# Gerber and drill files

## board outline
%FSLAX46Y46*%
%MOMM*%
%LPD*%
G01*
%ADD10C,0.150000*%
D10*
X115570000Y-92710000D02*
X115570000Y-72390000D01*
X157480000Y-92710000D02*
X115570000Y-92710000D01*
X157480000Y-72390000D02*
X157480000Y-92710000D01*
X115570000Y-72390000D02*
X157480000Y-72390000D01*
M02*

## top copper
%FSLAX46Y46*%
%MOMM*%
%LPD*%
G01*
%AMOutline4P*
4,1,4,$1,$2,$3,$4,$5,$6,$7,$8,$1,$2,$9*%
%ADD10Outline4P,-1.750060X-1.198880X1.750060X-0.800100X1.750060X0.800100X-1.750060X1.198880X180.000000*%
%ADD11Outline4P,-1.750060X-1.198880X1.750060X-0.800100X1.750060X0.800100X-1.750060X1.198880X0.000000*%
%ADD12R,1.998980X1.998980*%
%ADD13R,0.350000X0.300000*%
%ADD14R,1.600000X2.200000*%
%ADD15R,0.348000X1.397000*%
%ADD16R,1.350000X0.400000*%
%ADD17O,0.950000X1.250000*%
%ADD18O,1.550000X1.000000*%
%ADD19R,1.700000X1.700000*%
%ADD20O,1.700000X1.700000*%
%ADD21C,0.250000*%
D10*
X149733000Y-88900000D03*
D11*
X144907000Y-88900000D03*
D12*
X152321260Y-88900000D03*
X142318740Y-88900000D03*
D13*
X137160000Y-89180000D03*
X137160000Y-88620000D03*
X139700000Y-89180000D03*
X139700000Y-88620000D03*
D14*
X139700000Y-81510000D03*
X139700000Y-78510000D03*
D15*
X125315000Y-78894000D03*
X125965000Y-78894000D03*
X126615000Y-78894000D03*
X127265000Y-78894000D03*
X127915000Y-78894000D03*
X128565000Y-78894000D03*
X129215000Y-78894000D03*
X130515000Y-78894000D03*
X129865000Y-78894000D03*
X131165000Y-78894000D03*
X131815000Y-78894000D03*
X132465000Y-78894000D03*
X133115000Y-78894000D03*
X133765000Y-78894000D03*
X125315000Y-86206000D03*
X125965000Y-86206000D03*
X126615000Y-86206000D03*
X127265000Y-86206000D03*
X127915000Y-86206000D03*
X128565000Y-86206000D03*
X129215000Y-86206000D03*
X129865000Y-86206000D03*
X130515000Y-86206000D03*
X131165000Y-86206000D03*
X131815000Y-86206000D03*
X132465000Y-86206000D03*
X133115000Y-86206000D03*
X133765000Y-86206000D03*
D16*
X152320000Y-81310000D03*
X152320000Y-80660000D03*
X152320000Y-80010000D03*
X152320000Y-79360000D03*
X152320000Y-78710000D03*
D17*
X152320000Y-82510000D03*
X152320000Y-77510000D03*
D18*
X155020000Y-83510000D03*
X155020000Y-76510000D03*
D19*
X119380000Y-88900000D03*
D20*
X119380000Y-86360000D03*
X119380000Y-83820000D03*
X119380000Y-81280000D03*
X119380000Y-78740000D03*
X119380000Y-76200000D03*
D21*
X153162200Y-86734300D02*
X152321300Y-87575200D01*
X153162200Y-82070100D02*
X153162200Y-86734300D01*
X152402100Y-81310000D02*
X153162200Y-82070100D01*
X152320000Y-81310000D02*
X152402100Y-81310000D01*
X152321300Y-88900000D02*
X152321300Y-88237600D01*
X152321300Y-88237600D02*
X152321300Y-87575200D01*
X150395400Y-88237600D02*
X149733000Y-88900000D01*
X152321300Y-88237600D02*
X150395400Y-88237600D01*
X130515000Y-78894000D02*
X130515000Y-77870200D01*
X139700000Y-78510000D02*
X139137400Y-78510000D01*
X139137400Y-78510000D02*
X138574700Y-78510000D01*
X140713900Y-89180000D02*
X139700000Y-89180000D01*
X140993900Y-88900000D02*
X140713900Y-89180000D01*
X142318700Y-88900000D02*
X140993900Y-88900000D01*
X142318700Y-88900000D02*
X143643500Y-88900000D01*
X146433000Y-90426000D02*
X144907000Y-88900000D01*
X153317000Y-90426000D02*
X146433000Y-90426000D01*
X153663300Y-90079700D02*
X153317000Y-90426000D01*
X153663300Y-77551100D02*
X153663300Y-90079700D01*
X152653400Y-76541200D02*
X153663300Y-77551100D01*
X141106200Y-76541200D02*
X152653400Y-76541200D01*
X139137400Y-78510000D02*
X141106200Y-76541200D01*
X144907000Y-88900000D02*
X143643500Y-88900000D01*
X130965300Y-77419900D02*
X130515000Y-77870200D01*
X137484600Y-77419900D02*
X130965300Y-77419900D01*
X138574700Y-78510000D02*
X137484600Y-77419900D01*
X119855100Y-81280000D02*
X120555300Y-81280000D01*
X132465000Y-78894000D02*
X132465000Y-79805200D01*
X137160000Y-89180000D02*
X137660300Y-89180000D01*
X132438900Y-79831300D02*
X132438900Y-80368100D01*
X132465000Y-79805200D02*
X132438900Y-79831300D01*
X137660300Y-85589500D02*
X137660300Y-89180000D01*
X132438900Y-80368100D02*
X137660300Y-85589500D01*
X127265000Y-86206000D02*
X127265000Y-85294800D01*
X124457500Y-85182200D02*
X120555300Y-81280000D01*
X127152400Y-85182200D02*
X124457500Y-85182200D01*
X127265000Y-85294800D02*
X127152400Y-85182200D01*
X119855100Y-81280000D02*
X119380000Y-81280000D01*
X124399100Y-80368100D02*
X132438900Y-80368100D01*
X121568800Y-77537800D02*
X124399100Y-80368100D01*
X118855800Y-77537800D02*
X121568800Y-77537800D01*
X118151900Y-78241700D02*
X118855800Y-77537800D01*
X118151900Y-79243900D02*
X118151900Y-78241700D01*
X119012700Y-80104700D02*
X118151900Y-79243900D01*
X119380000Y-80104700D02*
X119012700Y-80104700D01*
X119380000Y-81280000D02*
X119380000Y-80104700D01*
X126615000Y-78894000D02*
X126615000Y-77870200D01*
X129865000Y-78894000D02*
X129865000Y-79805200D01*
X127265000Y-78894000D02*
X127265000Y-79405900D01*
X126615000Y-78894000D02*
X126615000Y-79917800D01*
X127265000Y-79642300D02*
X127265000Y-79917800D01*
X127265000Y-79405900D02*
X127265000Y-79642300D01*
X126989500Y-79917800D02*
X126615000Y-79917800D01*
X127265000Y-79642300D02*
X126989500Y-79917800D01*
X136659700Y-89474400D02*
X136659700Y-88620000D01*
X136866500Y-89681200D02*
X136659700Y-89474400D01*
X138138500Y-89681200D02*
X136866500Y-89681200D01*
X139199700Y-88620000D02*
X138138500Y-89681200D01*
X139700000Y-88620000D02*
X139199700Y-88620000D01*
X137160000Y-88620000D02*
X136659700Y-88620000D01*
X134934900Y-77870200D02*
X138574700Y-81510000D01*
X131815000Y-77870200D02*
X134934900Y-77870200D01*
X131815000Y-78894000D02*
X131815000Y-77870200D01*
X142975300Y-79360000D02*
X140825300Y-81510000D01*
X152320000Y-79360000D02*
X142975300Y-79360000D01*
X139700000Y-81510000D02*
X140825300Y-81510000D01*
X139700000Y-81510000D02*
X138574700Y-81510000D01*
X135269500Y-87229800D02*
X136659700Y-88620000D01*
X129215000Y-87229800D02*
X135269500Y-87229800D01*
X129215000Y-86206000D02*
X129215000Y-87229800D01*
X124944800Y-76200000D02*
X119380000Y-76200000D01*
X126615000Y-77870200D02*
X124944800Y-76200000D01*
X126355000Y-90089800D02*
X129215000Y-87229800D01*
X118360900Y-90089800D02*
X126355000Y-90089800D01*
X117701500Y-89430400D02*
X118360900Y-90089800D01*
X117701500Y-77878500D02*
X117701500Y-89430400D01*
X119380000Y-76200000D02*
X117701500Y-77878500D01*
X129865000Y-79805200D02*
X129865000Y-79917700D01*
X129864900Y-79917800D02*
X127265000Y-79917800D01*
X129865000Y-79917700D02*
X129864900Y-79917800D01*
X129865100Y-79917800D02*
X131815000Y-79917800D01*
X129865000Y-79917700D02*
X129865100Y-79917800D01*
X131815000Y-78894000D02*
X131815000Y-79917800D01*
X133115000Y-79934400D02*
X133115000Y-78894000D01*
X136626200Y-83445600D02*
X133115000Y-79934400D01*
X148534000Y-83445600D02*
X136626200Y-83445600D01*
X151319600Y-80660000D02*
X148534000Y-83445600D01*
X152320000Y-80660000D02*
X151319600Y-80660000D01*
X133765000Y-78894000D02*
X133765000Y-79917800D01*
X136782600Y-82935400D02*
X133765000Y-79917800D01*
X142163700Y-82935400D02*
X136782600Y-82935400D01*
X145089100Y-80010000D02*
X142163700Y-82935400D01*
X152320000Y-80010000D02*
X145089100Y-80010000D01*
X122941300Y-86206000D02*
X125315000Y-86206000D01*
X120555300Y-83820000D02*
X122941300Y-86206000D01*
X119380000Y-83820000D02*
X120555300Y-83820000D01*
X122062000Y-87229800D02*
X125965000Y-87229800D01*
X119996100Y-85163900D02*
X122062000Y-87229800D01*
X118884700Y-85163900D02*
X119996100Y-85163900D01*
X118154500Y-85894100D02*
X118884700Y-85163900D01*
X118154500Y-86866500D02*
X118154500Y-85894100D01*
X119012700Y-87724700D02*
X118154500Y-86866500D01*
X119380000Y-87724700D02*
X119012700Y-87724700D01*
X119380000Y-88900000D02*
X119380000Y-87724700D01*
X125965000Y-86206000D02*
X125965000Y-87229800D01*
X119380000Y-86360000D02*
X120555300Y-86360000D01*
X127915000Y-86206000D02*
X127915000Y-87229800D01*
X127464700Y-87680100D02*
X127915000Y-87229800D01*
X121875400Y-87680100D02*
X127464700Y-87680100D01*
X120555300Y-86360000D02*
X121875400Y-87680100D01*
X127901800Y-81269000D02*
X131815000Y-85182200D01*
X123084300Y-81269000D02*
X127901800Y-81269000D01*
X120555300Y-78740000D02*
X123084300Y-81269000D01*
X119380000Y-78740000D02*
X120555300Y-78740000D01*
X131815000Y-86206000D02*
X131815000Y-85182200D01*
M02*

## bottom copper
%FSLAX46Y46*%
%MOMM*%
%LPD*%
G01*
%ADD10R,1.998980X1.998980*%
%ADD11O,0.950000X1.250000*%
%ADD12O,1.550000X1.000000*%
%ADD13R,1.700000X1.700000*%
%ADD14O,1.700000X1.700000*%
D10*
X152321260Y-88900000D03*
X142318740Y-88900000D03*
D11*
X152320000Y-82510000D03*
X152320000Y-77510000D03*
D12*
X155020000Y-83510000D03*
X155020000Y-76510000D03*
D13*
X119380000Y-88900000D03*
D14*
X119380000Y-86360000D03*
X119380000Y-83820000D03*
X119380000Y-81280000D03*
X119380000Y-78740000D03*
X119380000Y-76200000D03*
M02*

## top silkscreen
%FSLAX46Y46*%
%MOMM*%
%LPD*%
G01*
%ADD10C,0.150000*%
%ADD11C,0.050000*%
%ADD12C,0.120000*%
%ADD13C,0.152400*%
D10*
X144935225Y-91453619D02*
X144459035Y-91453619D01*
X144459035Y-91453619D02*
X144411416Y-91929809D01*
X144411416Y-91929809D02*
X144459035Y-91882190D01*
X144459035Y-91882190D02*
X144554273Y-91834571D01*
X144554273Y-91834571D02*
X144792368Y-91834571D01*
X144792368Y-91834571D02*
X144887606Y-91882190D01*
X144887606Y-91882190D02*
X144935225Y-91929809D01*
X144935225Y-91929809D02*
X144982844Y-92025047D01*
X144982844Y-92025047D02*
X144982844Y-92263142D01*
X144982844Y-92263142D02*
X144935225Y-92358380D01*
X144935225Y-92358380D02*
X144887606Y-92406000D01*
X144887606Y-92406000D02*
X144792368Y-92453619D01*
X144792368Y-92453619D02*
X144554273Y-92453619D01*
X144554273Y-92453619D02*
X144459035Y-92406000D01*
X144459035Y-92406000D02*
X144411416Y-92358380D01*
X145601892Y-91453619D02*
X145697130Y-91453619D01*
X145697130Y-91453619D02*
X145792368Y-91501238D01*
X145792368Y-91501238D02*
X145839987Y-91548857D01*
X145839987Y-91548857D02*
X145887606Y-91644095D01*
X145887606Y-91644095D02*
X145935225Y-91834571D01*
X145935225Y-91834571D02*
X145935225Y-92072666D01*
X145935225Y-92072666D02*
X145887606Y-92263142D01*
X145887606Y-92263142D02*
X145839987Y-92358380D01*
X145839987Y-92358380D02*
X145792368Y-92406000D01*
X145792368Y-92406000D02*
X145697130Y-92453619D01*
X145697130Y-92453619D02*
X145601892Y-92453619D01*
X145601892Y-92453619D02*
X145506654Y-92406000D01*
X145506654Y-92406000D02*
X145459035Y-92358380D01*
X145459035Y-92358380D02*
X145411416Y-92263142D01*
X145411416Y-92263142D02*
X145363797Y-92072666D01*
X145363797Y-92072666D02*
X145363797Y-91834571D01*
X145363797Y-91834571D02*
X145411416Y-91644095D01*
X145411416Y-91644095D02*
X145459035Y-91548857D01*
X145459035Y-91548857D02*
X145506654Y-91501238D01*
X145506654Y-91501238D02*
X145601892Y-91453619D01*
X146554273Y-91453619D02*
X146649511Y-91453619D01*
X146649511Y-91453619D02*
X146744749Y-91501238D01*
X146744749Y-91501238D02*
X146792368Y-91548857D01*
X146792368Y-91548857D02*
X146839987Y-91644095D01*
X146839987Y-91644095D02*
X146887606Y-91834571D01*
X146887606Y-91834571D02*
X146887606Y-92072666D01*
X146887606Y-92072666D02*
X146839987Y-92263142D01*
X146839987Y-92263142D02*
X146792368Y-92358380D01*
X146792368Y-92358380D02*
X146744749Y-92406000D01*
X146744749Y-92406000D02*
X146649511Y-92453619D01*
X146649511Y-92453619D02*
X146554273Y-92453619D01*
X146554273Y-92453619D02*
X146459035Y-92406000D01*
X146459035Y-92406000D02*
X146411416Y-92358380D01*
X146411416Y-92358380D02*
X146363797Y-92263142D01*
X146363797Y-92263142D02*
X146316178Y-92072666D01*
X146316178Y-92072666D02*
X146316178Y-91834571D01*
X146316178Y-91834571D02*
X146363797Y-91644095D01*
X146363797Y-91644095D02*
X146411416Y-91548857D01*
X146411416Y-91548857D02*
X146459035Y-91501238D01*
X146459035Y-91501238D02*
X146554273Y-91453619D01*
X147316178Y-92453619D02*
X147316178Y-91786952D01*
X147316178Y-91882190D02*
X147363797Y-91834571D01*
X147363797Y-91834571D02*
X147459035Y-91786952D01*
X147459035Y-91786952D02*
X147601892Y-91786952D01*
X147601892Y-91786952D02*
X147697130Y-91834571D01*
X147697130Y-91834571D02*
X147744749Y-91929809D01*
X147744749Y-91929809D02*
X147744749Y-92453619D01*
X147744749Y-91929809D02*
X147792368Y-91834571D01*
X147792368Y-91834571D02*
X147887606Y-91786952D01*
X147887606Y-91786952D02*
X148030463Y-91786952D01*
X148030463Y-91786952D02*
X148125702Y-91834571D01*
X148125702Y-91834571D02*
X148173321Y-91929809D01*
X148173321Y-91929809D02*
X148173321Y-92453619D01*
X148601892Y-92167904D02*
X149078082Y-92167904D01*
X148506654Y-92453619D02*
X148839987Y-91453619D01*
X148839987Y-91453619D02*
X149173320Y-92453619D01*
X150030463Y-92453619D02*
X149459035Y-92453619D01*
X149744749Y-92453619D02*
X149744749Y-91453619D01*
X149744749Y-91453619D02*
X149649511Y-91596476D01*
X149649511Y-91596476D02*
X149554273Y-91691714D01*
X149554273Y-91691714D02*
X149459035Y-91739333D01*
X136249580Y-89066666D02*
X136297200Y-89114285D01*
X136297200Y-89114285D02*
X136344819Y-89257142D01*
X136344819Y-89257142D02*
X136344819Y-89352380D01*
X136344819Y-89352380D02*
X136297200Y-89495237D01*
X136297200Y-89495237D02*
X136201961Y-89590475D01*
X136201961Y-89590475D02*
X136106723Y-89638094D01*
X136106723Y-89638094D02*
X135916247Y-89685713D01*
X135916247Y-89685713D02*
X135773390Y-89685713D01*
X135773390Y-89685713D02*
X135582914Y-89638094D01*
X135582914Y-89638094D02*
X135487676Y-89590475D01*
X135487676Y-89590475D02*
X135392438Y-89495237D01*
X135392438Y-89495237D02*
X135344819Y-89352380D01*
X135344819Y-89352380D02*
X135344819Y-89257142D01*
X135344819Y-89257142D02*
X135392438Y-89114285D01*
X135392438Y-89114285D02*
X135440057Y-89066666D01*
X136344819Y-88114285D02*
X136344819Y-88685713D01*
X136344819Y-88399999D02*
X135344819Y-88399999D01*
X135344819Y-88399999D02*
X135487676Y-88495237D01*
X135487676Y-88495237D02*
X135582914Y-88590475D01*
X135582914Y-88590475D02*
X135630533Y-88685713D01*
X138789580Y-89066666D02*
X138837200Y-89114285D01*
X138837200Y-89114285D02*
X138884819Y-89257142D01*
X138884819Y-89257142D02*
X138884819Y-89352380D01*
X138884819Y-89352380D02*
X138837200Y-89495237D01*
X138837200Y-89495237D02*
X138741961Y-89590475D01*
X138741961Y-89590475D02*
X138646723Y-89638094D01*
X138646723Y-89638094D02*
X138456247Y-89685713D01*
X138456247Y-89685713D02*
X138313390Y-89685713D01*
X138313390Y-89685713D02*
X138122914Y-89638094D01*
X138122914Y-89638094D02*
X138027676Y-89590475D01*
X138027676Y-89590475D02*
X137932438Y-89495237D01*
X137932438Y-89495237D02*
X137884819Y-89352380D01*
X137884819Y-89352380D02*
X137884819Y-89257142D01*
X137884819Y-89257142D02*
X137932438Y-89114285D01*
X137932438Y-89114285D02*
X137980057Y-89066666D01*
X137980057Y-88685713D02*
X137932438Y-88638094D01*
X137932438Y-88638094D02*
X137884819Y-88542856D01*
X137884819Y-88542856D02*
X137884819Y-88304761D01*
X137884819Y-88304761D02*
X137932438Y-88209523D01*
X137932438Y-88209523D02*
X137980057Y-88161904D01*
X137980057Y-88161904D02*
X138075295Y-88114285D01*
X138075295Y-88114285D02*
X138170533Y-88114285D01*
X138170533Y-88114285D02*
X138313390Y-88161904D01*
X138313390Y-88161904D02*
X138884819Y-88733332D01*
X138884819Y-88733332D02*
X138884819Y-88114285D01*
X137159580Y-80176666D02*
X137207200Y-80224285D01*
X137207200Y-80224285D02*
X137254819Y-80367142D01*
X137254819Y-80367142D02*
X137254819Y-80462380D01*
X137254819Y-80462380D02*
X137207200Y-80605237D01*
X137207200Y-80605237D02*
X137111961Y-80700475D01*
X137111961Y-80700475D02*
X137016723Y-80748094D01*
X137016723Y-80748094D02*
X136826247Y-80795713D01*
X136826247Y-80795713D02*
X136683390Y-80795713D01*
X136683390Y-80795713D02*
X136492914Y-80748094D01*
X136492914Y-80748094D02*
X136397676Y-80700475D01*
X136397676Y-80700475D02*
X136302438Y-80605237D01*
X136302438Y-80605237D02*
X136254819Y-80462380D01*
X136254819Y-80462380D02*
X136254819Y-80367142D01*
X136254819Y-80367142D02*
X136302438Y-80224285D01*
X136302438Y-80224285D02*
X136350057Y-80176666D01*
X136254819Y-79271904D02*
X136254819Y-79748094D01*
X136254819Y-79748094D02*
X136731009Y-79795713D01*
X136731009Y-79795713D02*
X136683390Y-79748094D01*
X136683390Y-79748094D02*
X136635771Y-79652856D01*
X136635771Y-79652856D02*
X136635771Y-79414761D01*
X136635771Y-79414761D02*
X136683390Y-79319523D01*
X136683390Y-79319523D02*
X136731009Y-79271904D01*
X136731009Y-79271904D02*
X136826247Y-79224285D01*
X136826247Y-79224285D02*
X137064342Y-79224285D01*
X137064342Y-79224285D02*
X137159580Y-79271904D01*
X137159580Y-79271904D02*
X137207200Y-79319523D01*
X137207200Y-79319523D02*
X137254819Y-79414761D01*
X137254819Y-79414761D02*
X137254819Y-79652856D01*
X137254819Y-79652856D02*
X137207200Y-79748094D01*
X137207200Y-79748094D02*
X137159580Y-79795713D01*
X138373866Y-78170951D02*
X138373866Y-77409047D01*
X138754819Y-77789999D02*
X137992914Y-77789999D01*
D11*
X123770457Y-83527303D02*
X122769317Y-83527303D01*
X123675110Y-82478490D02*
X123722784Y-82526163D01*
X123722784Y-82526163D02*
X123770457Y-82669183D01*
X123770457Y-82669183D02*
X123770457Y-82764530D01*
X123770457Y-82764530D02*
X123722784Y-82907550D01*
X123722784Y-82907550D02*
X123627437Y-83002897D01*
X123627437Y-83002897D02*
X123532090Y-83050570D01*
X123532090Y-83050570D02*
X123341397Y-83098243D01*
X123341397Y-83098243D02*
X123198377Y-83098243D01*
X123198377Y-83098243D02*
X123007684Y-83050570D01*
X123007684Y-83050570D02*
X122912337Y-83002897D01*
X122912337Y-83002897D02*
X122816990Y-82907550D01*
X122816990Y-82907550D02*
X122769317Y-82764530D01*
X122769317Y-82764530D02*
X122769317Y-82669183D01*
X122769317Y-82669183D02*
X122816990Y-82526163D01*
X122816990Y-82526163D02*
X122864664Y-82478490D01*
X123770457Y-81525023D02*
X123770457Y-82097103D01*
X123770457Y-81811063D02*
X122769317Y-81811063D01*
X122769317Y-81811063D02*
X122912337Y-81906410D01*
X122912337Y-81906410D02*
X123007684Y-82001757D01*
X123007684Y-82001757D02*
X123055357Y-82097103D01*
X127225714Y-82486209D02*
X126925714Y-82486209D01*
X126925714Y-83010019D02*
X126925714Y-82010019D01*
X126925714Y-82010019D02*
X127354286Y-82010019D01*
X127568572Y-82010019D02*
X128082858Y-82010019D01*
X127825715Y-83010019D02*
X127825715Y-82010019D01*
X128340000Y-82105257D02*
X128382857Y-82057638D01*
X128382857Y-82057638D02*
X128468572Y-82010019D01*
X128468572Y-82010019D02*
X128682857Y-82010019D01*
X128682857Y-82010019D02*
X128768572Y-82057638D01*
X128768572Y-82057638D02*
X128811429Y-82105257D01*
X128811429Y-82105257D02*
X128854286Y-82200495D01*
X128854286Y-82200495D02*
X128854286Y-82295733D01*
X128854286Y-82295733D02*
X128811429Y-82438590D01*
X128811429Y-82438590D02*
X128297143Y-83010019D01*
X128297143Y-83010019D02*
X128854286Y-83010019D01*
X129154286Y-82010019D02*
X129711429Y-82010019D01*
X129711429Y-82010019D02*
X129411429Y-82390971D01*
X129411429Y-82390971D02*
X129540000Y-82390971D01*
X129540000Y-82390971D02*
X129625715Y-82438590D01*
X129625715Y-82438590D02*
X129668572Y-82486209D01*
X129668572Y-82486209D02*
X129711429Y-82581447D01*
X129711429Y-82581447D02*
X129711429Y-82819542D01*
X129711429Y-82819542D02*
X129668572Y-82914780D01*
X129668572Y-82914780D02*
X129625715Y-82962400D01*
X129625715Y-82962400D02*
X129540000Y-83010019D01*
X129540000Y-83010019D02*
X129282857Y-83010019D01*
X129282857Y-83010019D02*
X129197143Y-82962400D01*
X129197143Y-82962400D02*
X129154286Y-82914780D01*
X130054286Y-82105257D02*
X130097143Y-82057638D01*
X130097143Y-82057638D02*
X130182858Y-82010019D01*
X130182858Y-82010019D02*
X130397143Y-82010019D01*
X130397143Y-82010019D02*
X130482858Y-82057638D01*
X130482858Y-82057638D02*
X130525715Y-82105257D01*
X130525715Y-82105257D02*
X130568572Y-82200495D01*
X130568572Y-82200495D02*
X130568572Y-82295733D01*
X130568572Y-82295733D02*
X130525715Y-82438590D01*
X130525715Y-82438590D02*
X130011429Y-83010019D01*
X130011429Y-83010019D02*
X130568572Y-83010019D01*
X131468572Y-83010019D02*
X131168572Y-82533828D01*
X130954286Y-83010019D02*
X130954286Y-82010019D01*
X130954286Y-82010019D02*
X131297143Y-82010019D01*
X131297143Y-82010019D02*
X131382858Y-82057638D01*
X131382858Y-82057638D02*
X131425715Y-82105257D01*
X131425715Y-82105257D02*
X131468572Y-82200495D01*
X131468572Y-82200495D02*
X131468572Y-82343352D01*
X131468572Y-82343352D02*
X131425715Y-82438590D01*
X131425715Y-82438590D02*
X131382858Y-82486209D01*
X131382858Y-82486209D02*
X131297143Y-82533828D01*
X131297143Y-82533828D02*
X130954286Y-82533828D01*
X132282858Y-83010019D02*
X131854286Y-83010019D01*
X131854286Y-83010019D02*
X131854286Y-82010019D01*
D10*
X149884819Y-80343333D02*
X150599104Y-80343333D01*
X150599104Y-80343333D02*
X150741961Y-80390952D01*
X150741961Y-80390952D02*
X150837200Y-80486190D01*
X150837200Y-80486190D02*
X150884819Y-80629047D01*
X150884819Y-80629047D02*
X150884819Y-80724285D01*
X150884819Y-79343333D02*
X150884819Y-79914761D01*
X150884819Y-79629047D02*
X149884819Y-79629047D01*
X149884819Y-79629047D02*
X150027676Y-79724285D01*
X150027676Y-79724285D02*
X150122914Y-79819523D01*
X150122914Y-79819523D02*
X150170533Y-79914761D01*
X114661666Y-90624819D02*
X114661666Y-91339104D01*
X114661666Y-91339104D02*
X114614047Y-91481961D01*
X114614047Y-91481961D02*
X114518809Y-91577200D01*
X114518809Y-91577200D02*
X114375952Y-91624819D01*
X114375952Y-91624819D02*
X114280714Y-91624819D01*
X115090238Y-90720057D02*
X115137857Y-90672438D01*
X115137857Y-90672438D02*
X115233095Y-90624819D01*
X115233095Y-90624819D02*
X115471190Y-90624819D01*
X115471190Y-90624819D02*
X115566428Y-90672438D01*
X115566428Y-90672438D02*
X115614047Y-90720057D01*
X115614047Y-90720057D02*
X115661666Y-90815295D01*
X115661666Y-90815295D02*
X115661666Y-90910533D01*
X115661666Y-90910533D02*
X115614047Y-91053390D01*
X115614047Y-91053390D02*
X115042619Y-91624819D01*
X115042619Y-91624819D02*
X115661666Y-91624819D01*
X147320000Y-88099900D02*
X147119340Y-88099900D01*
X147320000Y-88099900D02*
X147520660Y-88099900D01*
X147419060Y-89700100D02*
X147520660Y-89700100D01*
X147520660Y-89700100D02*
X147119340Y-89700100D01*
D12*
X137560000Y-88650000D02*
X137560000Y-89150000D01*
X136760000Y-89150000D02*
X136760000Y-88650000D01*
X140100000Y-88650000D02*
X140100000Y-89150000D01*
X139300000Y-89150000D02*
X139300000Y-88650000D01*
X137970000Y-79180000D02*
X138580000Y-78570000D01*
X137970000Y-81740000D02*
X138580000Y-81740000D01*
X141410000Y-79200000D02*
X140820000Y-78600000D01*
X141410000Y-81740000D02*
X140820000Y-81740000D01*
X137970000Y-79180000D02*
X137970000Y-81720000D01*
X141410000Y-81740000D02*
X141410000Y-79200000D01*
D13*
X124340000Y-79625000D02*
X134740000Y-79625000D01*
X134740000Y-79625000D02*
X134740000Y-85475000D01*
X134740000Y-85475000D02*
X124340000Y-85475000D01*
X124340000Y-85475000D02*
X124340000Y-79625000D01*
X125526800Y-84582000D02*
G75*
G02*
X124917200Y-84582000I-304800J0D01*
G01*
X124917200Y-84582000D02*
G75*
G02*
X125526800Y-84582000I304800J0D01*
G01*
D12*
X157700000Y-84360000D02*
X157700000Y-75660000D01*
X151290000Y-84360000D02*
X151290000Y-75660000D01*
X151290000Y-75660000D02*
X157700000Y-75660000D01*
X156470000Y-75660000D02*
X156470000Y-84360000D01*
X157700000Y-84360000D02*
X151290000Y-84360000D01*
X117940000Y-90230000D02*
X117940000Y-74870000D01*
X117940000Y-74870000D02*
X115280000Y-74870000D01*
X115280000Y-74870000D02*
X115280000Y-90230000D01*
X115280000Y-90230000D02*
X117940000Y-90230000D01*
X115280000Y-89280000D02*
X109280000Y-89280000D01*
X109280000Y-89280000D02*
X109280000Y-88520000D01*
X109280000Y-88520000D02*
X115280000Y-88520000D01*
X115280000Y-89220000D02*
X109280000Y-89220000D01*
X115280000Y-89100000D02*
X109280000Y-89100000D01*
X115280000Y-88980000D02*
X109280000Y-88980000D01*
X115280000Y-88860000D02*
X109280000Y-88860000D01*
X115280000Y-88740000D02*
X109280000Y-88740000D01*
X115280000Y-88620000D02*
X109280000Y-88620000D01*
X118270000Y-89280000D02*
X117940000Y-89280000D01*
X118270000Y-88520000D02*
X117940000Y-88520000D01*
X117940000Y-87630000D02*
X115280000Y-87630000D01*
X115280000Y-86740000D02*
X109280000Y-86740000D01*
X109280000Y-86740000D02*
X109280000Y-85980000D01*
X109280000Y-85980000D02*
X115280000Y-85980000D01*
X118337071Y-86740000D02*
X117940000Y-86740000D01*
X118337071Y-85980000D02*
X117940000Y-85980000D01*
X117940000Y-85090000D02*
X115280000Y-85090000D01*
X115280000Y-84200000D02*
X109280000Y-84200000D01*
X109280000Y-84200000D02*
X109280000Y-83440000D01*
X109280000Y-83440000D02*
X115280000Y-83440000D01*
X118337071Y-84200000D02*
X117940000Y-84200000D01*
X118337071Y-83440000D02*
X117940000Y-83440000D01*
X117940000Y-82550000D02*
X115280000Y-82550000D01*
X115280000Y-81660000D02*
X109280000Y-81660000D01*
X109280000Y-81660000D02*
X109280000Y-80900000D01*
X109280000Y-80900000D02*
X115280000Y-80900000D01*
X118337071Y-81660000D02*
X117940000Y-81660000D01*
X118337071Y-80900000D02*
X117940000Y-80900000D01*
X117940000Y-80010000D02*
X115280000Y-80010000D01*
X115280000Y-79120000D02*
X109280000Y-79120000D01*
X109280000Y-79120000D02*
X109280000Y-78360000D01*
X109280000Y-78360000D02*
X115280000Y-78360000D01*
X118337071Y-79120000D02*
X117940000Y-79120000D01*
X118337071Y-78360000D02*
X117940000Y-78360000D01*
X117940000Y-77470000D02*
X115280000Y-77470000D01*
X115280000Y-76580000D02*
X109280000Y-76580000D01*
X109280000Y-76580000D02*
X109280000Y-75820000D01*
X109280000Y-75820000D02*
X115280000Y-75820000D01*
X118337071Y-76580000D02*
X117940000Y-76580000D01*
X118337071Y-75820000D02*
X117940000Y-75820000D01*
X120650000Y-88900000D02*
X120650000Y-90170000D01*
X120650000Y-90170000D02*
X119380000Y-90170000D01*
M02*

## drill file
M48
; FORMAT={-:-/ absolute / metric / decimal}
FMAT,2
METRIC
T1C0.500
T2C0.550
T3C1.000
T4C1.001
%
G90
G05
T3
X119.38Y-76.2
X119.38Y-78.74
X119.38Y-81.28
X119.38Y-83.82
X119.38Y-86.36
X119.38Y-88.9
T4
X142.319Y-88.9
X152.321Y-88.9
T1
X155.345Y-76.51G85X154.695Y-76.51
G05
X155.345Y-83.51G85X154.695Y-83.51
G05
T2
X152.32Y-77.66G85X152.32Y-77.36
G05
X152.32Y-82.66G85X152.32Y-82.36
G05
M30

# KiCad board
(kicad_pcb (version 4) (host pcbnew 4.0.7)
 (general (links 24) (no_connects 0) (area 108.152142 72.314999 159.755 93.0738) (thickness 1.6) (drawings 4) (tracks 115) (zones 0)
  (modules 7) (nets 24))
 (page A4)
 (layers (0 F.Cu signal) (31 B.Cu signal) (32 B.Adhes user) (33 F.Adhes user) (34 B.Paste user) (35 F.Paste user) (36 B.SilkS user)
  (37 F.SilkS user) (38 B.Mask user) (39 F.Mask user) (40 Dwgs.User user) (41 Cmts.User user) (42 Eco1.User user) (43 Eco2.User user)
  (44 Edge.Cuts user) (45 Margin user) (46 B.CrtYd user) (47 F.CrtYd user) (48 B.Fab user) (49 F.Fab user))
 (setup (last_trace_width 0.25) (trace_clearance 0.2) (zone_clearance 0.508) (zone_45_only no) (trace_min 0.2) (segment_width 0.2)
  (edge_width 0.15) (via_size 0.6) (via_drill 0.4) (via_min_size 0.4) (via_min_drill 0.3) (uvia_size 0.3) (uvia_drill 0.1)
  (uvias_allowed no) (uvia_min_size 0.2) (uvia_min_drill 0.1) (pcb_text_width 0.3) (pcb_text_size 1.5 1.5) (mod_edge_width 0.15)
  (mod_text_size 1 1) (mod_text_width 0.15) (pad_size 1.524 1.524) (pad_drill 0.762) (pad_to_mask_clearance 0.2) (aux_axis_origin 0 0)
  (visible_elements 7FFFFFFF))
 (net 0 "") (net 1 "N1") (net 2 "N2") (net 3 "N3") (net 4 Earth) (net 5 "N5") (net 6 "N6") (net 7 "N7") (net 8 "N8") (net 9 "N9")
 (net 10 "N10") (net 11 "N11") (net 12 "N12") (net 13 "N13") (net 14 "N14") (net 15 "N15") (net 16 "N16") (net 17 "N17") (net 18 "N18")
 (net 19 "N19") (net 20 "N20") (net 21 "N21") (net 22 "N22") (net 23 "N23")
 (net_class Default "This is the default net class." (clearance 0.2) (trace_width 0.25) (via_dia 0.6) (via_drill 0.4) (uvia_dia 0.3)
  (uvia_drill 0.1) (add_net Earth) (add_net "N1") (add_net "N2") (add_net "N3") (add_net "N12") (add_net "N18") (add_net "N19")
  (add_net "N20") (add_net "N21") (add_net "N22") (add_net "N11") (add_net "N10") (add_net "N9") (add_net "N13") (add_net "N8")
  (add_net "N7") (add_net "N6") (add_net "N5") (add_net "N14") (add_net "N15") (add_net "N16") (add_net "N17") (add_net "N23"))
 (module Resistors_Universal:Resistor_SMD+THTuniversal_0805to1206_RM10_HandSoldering (layer F.Cu) (at 147.32 88.9 180)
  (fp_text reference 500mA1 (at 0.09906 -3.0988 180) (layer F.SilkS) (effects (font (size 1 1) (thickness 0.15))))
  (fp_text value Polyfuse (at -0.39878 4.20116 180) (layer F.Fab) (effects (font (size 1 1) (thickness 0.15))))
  (fp_line (start 0 0.8001) (end 0.20066 0.8001) (layer F.SilkS) (width 0.15))
  (fp_line (start 0 0.8001) (end -0.20066 0.8001) (layer F.SilkS) (width 0.15))
  (fp_line (start -0.09906 -0.8001) (end -0.20066 -0.8001) (layer F.SilkS) (width 0.15))
  (fp_line (start -0.20066 -0.8001) (end 0.20066 -0.8001) (layer F.SilkS) (width 0.15))
  (pad 1 smd trapezoid (at -2.413 0 180) (size 3.50012 1.99898) (rect_delta 0.39878 0) (layers F.Cu F.Paste F.Mask) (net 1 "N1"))
  (pad 2 smd trapezoid (at 2.413 0) (size 3.50012 1.99898) (rect_delta 0.39878 0) (layers F.Cu F.Paste F.Mask) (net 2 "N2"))
  (pad 1 thru_hole rect (at -5.00126 0) (size 1.99898 1.99898) (drill 1.00076) (layers *.Cu *.Mask) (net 1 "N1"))
  (pad 2 thru_hole rect (at 5.00126 0) (size 1.99898 1.99898) (drill 1.00076) (layers *.Cu *.Mask) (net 2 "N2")))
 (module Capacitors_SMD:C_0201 (layer F.Cu) (at 137.16 88.9 90)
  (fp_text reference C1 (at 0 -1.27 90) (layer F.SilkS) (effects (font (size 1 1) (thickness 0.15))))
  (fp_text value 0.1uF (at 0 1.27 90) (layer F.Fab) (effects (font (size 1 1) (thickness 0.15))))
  (fp_line (start 0.25 0.4) (end -0.25 0.4) (layer F.SilkS) (width 0.12))
  (fp_line (start -0.25 -0.4) (end 0.25 -0.4) (layer F.SilkS) (width 0.12))
  (pad 1 smd rect (at -0.28 0 90) (size 0.3 0.35) (layers F.Cu F.Paste F.Mask) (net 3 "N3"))
  (pad 2 smd rect (at 0.28 0 90) (size 0.3 0.35) (layers F.Cu F.Paste F.Mask) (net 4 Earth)))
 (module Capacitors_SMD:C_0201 (layer F.Cu) (at 139.7 88.9 90)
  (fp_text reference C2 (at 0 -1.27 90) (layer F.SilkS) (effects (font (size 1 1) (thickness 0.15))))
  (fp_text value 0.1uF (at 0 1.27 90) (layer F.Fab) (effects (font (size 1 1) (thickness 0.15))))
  (fp_line (start 0.25 0.4) (end -0.25 0.4) (layer F.SilkS) (width 0.12))
  (fp_line (start -0.25 -0.4) (end 0.25 -0.4) (layer F.SilkS) (width 0.12))
  (pad 1 smd rect (at -0.28 0 90) (size 0.3 0.35) (layers F.Cu F.Paste F.Mask) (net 2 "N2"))
  (pad 2 smd rect (at 0.28 0 90) (size 0.3 0.35) (layers F.Cu F.Paste F.Mask) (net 4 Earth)))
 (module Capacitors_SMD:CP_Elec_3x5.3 (layer F.Cu) (at 139.7 80.01 270)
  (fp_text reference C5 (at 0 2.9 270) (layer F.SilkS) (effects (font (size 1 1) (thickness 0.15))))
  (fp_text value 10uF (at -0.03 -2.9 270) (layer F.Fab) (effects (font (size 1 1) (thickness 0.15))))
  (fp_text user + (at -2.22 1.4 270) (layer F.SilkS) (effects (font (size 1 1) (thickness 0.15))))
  (fp_line (start -0.83 1.73) (end -1.44 1.12) (layer F.SilkS) (width 0.12))
  (fp_line (start 1.73 1.73) (end 1.73 1.12) (layer F.SilkS) (width 0.12))
  (fp_line (start -0.81 -1.71) (end -1.41 -1.12) (layer F.SilkS) (width 0.12))
  (fp_line (start 1.73 -1.71) (end 1.73 -1.12) (layer F.SilkS) (width 0.12))
  (fp_line (start -0.83 1.73) (end 1.71 1.73) (layer F.SilkS) (width 0.12))
  (fp_line (start 1.73 -1.71) (end -0.81 -1.71) (layer F.SilkS) (width 0.12))
  (pad 2 smd rect (at 1.5 0 270) (size 2.2 1.6) (layers F.Cu F.Paste F.Mask) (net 4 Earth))
  (pad 1 smd rect (at -1.5 0 270) (size 2.2 1.6) (layers F.Cu F.Paste F.Mask) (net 2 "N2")))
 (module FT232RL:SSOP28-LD (layer F.Cu) (at 129.54 82.55)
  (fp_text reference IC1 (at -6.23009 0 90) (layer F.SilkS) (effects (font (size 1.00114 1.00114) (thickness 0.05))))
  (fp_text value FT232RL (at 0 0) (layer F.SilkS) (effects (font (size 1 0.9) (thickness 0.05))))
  (fp_line (start -5.2 -2.925) (end 5.2 -2.925) (layer F.SilkS) (width 0.1524))
  (fp_line (start 5.2 -2.925) (end 5.2 2.925) (layer F.SilkS) (width 0.1524))
  (fp_line (start 5.2 2.925) (end -5.2 2.925) (layer F.SilkS) (width 0.1524))
  (fp_line (start -5.2 2.925) (end -5.2 -2.925) (layer F.SilkS) (width 0.1524))
  (fp_circle (center -4.318 2.032) (end -4.0132 2.032) (layer F.SilkS) (width 0.1524))
  (pad 28 smd rect (at -4.225 -3.656) (size 0.348 1.397) (layers F.Cu F.Paste F.Mask) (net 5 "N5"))
  (pad 27 smd rect (at -3.575 -3.656) (size 0.348 1.397) (layers F.Cu F.Paste F.Mask) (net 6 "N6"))
  (pad 26 smd rect (at -2.925 -3.656) (size 0.348 1.397) (layers F.Cu F.Paste F.Mask) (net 4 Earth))
  (pad 25 smd rect (at -2.275 -3.656) (size 0.348 1.397) (layers F.Cu F.Paste F.Mask) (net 4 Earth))
  (pad 24 smd rect (at -1.625 -3.656) (size 0.348 1.397) (layers F.Cu F.Paste F.Mask))
  (pad 23 smd rect (at -0.975 -3.656) (size 0.348 1.397) (layers F.Cu F.Paste F.Mask) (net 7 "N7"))
  (pad 22 smd rect (at -0.325 -3.656) (size 0.348 1.397) (layers F.Cu F.Paste F.Mask) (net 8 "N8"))
  (pad 20 smd rect (at 0.975 -3.656) (size 0.348 1.397) (layers F.Cu F.Paste F.Mask) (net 2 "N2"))
  (pad 21 smd rect (at 0.325 -3.656) (size 0.348 1.397) (layers F.Cu F.Paste F.Mask) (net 4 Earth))
  (pad 19 smd rect (at 1.625 -3.656) (size 0.348 1.397) (layers F.Cu F.Paste F.Mask) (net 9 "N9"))
  (pad 18 smd rect (at 2.275 -3.656) (size 0.348 1.397) (layers F.Cu F.Paste F.Mask) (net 4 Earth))
  (pad 17 smd rect (at 2.925 -3.656) (size 0.348 1.397) (layers F.Cu F.Paste F.Mask) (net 3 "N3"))
  (pad 16 smd rect (at 3.575 -3.656) (size 0.348 1.397) (layers F.Cu F.Paste F.Mask) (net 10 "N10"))
  (pad 15 smd rect (at 4.225 -3.656) (size 0.348 1.397) (layers F.Cu F.Paste F.Mask) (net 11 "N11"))
  (pad 1 smd rect (at -4.225 3.656) (size 0.348 1.397) (layers F.Cu F.Paste F.Mask) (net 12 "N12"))
  (pad 2 smd rect (at -3.575 3.656) (size 0.348 1.397) (layers F.Cu F.Paste F.Mask) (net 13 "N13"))
  (pad 3 smd rect (at -2.925 3.656) (size 0.348 1.397) (layers F.Cu F.Paste F.Mask) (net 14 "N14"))
  (pad 4 smd rect (at -2.275 3.656) (size 0.348 1.397) (layers F.Cu F.Paste F.Mask) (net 3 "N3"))
  (pad 5 smd rect (at -1.625 3.656) (size 0.348 1.397) (layers F.Cu F.Paste F.Mask) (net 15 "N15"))
  (pad 6 smd rect (at -0.975 3.656) (size 0.348 1.397) (layers F.Cu F.Paste F.Mask) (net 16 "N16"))
  (pad 7 smd rect (at -0.325 3.656) (size 0.348 1.397) (layers F.Cu F.Paste F.Mask) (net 4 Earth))
  (pad 8 smd rect (at 0.325 3.656) (size 0.348 1.397) (layers F.Cu F.Paste F.Mask))
  (pad 9 smd rect (at 0.975 3.656) (size 0.348 1.397) (layers F.Cu F.Paste F.Mask) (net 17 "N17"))
  (pad 10 smd rect (at 1.625 3.656) (size 0.348 1.397) (layers F.Cu F.Paste F.Mask) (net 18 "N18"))
  (pad 11 smd rect (at 2.275 3.656) (size 0.348 1.397) (layers F.Cu F.Paste F.Mask) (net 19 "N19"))
  (pad 12 smd rect (at 2.925 3.656) (size 0.348 1.397) (layers F.Cu F.Paste F.Mask) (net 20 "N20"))
  (pad 13 smd rect (at 3.575 3.656) (size 0.348 1.397) (layers F.Cu F.Paste F.Mask) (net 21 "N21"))
  (pad 14 smd rect (at 4.225 3.656) (size 0.348 1.397) (layers F.Cu F.Paste F.Mask) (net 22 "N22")))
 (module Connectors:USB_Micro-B (layer F.Cu) (at 153.67 80.01 90)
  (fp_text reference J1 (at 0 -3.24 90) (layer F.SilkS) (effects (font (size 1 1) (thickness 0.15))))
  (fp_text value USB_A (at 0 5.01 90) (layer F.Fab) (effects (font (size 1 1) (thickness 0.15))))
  (fp_line (start -4.35 4.03) (end 4.35 4.03) (layer F.SilkS) (width 0.12))
  (fp_line (start -4.35 -2.38) (end 4.35 -2.38) (layer F.SilkS) (width 0.12))
  (fp_line (start 4.35 -2.38) (end 4.35 4.03) (layer F.SilkS) (width 0.12))
  (fp_line (start 4.35 2.8) (end -4.35 2.8) (layer F.SilkS) (width 0.12))
  (fp_line (start -4.35 4.03) (end -4.35 -2.38) (layer F.SilkS) (width 0.12))
  (pad 1 smd rect (at -1.3 -1.35 180) (size 1.35 0.4) (layers F.Cu F.Paste F.Mask) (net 1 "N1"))
  (pad 2 smd rect (at -0.65 -1.35 180) (size 1.35 0.4) (layers F.Cu F.Paste F.Mask) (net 10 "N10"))
  (pad 3 smd rect (at 0 -1.35 180) (size 1.35 0.4) (layers F.Cu F.Paste F.Mask) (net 11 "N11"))
  (pad 4 smd rect (at 0.65 -1.35 180) (size 1.35 0.4) (layers F.Cu F.Paste F.Mask) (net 4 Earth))
  (pad 5 smd rect (at 1.3 -1.35 180) (size 1.35 0.4) (layers F.Cu F.Paste F.Mask) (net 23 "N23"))
  (pad 6 thru_hole oval (at -2.5 -1.35 180) (size 0.95 1.25) (drill oval 0.55 0.85) (layers *.Cu *.Mask))
  (pad 6 thru_hole oval (at 2.5 -1.35 180) (size 0.95 1.25) (drill oval 0.55 0.85) (layers *.Cu *.Mask))
  (pad 6 thru_hole oval (at -3.5 1.35 180) (size 1.55 1) (drill oval 1.15 0.5) (layers *.Cu *.Mask))
  (pad 6 thru_hole oval (at 3.5 1.35 180) (size 1.55 1) (drill oval 1.15 0.5) (layers *.Cu *.Mask)))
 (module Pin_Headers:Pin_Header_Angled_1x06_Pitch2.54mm (layer F.Cu) (at 119.38 88.9 180)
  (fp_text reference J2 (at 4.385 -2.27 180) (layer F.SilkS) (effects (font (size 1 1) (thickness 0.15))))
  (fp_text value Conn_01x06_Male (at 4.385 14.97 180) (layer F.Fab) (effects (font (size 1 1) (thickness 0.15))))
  (fp_line (start 1.44 -1.33) (end 1.44 14.03) (layer F.SilkS) (width 0.12))
  (fp_line (start 1.44 14.03) (end 4.1 14.03) (layer F.SilkS) (width 0.12))
  (fp_line (start 4.1 14.03) (end 4.1 -1.33) (layer F.SilkS) (width 0.12))
  (fp_line (start 4.1 -1.33) (end 1.44 -1.33) (layer F.SilkS) (width 0.12))
  (fp_line (start 4.1 -0.38) (end 10.1 -0.38) (layer F.SilkS) (width 0.12))
  (fp_line (start 10.1 -0.38) (end 10.1 0.38) (layer F.SilkS) (width 0.12))
  (fp_line (start 10.1 0.38) (end 4.1 0.38) (layer F.SilkS) (width 0.12))
  (fp_line (start 4.1 -0.32) (end 10.1 -0.32) (layer F.SilkS) (width 0.12))
  (fp_line (start 4.1 -0.2) (end 10.1 -0.2) (layer F.SilkS) (width 0.12))
  (fp_line (start 4.1 -0.08) (end 10.1 -0.08) (layer F.SilkS) (width 0.12))
  (fp_line (start 4.1 0.04) (end 10.1 0.04) (layer F.SilkS) (width 0.12))
  (fp_line (start 4.1 0.16) (end 10.1 0.16) (layer F.SilkS) (width 0.12))
  (fp_line (start 4.1 0.28) (end 10.1 0.28) (layer F.SilkS) (width 0.12))
  (fp_line (start 1.11 -0.38) (end 1.44 -0.38) (layer F.SilkS) (width 0.12))
  (fp_line (start 1.11 0.38) (end 1.44 0.38) (layer F.SilkS) (width 0.12))
  (fp_line (start 1.44 1.27) (end 4.1 1.27) (layer F.SilkS) (width 0.12))
  (fp_line (start 4.1 2.16) (end 10.1 2.16) (layer F.SilkS) (width 0.12))
  (fp_line (start 10.1 2.16) (end 10.1 2.92) (layer F.SilkS) (width 0.12))
  (fp_line (start 10.1 2.92) (end 4.1 2.92) (layer F.SilkS) (width 0.12))
  (fp_line (start 1.042929 2.16) (end 1.44 2.16) (layer F.SilkS) (width 0.12))
  (fp_line (start 1.042929 2.92) (end 1.44 2.92) (layer F.SilkS) (width 0.12))
  (fp_line (start 1.44 3.81) (end 4.1 3.81) (layer F.SilkS) (width 0.12))
  (fp_line (start 4.1 4.7) (end 10.1 4.7) (layer F.SilkS) (width 0.12))
  (fp_line (start 10.1 4.7) (end 10.1 5.46) (layer F.SilkS) (width 0.12))
  (fp_line (start 10.1 5.46) (end 4.1 5.46) (layer F.SilkS) (width 0.12))
  (fp_line (start 1.042929 4.7) (end 1.44 4.7) (layer F.SilkS) (width 0.12))
  (fp_line (start 1.042929 5.46) (end 1.44 5.46) (layer F.SilkS) (width 0.12))
  (fp_line (start 1.44 6.35) (end 4.1 6.35) (layer F.SilkS) (width 0.12))
  (fp_line (start 4.1 7.24) (end 10.1 7.24) (layer F.SilkS) (width 0.12))
  (fp_line (start 10.1 7.24) (end 10.1 8) (layer F.SilkS) (width 0.12))
  (fp_line (start 10.1 8) (end 4.1 8) (layer F.SilkS) (width 0.12))
  (fp_line (start 1.042929 7.24) (end 1.44 7.24) (layer F.SilkS) (width 0.12))
  (fp_line (start 1.042929 8) (end 1.44 8) (layer F.SilkS) (width 0.12))
  (fp_line (start 1.44 8.89) (end 4.1 8.89) (layer F.SilkS) (width 0.12))
  (fp_line (start 4.1 9.78) (end 10.1 9.78) (layer F.SilkS) (width 0.12))
  (fp_line (start 10.1 9.78) (end 10.1 10.54) (layer F.SilkS) (width 0.12))
  (fp_line (start 10.1 10.54) (end 4.1 10.54) (layer F.SilkS) (width 0.12))
  (fp_line (start 1.042929 9.78) (end 1.44 9.78) (layer F.SilkS) (width 0.12))
  (fp_line (start 1.042929 10.54) (end 1.44 10.54) (layer F.SilkS) (width 0.12))
  (fp_line (start 1.44 11.43) (end 4.1 11.43) (layer F.SilkS) (width 0.12))
  (fp_line (start 4.1 12.32) (end 10.1 12.32) (layer F.SilkS) (width 0.12))
  (fp_line (start 10.1 12.32) (end 10.1 13.08) (layer F.SilkS) (width 0.12))
  (fp_line (start 10.1 13.08) (end 4.1 13.08) (layer F.SilkS) (width 0.12))
  (fp_line (start 1.042929 12.32) (end 1.44 12.32) (layer F.SilkS) (width 0.12))
  (fp_line (start 1.042929 13.08) (end 1.44 13.08) (layer F.SilkS) (width 0.12))
  (fp_line (start -1.27 0) (end -1.27 -1.27) (layer F.SilkS) (width 0.12))
  (fp_line (start -1.27 -1.27) (end 0 -1.27) (layer F.SilkS) (width 0.12))
  (pad 1 thru_hole rect (at 0 0 180) (size 1.7 1.7) (drill 1) (layers *.Cu *.Mask) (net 13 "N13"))
  (pad 2 thru_hole oval (at 0 2.54 180) (size 1.7 1.7) (drill 1) (layers *.Cu *.Mask) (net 15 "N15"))
  (pad 3 thru_hole oval (at 0 5.08 180) (size 1.7 1.7) (drill 1) (layers *.Cu *.Mask) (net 12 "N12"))
  (pad 4 thru_hole oval (at 0 7.62 180) (size 1.7 1.7) (drill 1) (layers *.Cu *.Mask) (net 3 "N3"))
  (pad 5 thru_hole oval (at 0 10.16 180) (size 1.7 1.7) (drill 1) (layers *.Cu *.Mask) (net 19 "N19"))
  (pad 6 thru_hole oval (at 0 12.7 180) (size 1.7 1.7) (drill 1) (layers *.Cu *.Mask) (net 4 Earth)))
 (gr_line (start 115.57 92.71) (end 115.57 72.39) (angle 90) (layer Edge.Cuts) (width 0.15))
 (gr_line (start 157.48 92.71) (end 115.57 92.71) (angle 90) (layer Edge.Cuts) (width 0.15))
 (gr_line (start 157.48 72.39) (end 157.48 92.71) (angle 90) (layer Edge.Cuts) (width 0.15))
 (gr_line (start 115.57 72.39) (end 157.48 72.39) (angle 90) (layer Edge.Cuts) (width 0.15))
 (segment (start 153.1622 86.7343) (end 152.3213 87.5752) (width 0.25) (layer F.Cu) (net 1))
 (segment (start 153.1622 82.0701) (end 153.1622 86.7343) (width 0.25) (layer F.Cu) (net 1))
 (segment (start 152.4021 81.31) (end 153.1622 82.0701) (width 0.25) (layer F.Cu) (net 1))
 (segment (start 152.32 81.31) (end 152.4021 81.31) (width 0.25) (layer F.Cu) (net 1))
 (segment (start 152.3213 88.9) (end 152.3213 88.2376) (width 0.25) (layer F.Cu) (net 1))
 (segment (start 152.3213 88.2376) (end 152.3213 87.5752) (width 0.25) (layer F.Cu) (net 1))
 (segment (start 150.3954 88.2376) (end 149.733 88.9) (width 0.25) (layer F.Cu) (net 1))
 (segment (start 152.3213 88.2376) (end 150.3954 88.2376) (width 0.25) (layer F.Cu) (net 1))
 (segment (start 130.515 78.894) (end 130.515 77.8702) (width 0.25) (layer F.Cu) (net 2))
 (segment (start 139.7 78.51) (end 139.1374 78.51) (width 0.25) (layer F.Cu) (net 2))
 (segment (start 139.1374 78.51) (end 138.5747 78.51) (width 0.25) (layer F.Cu) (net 2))
 (segment (start 140.7139 89.18) (end 139.7 89.18) (width 0.25) (layer F.Cu) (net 2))
 (segment (start 140.9939 88.9) (end 140.7139 89.18) (width 0.25) (layer F.Cu) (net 2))
 (segment (start 142.3187 88.9) (end 140.9939 88.9) (width 0.25) (layer F.Cu) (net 2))
 (segment (start 142.3187 88.9) (end 143.6435 88.9) (width 0.25) (layer F.Cu) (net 2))
 (segment (start 146.433 90.426) (end 144.907 88.9) (width 0.25) (layer F.Cu) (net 2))
 (segment (start 153.317 90.426) (end 146.433 90.426) (width 0.25) (layer F.Cu) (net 2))
 (segment (start 153.6633 90.0797) (end 153.317 90.426) (width 0.25) (layer F.Cu) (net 2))
 (segment (start 153.6633 77.5511) (end 153.6633 90.0797) (width 0.25) (layer F.Cu) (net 2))
 (segment (start 152.6534 76.5412) (end 153.6633 77.5511) (width 0.25) (layer F.Cu) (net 2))
 (segment (start 141.1062 76.5412) (end 152.6534 76.5412) (width 0.25) (layer F.Cu) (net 2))
 (segment (start 139.1374 78.51) (end 141.1062 76.5412) (width 0.25) (layer F.Cu) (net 2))
 (segment (start 144.907 88.9) (end 143.6435 88.9) (width 0.25) (layer F.Cu) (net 2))
 (segment (start 130.9653 77.4199) (end 130.515 77.8702) (width 0.25) (layer F.Cu) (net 2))
 (segment (start 137.4846 77.4199) (end 130.9653 77.4199) (width 0.25) (layer F.Cu) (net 2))
 (segment (start 138.5747 78.51) (end 137.4846 77.4199) (width 0.25) (layer F.Cu) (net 2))
 (segment (start 119.8551 81.28) (end 120.5553 81.28) (width 0.25) (layer F.Cu) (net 3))
 (segment (start 132.465 78.894) (end 132.465 79.8052) (width 0.25) (layer F.Cu) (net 3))
 (segment (start 137.16 89.18) (end 137.6603 89.18) (width 0.25) (layer F.Cu) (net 3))
 (segment (start 132.4389 79.8313) (end 132.4389 80.3681) (width 0.25) (layer F.Cu) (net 3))
 (segment (start 132.465 79.8052) (end 132.4389 79.8313) (width 0.25) (layer F.Cu) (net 3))
 (segment (start 137.6603 85.5895) (end 137.6603 89.18) (width 0.25) (layer F.Cu) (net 3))
 (segment (start 132.4389 80.3681) (end 137.6603 85.5895) (width 0.25) (layer F.Cu) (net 3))
 (segment (start 127.265 86.206) (end 127.265 85.2948) (width 0.25) (layer F.Cu) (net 3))
 (segment (start 124.4575 85.1822) (end 120.5553 81.28) (width 0.25) (layer F.Cu) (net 3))
 (segment (start 127.1524 85.1822) (end 124.4575 85.1822) (width 0.25) (layer F.Cu) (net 3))
 (segment (start 127.265 85.2948) (end 127.1524 85.1822) (width 0.25) (layer F.Cu) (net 3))
 (segment (start 119.8551 81.28) (end 119.38 81.28) (width 0.25) (layer F.Cu) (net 3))
 (segment (start 124.3991 80.3681) (end 132.4389 80.3681) (width 0.25) (layer F.Cu) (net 3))
 (segment (start 121.5688 77.5378) (end 124.3991 80.3681) (width 0.25) (layer F.Cu) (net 3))
 (segment (start 118.8558 77.5378) (end 121.5688 77.5378) (width 0.25) (layer F.Cu) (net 3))
 (segment (start 118.1519 78.2417) (end 118.8558 77.5378) (width 0.25) (layer F.Cu) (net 3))
 (segment (start 118.1519 79.2439) (end 118.1519 78.2417) (width 0.25) (layer F.Cu) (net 3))
 (segment (start 119.0127 80.1047) (end 118.1519 79.2439) (width 0.25) (layer F.Cu) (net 3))
 (segment (start 119.38 80.1047) (end 119.0127 80.1047) (width 0.25) (layer F.Cu) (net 3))
 (segment (start 119.38 81.28) (end 119.38 80.1047) (width 0.25) (layer F.Cu) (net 3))
 (segment (start 126.615 78.894) (end 126.615 77.8702) (width 0.25) (layer F.Cu) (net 4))
 (segment (start 129.865 78.894) (end 129.865 79.8052) (width 0.25) (layer F.Cu) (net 4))
 (segment (start 127.265 78.894) (end 127.265 79.4059) (width 0.25) (layer F.Cu) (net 4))
 (segment (start 126.615 78.894) (end 126.615 79.9178) (width 0.25) (layer F.Cu) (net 4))
 (segment (start 127.265 79.6423) (end 127.265 79.9178) (width 0.25) (layer F.Cu) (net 4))
 (segment (start 127.265 79.4059) (end 127.265 79.6423) (width 0.25) (layer F.Cu) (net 4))
 (segment (start 126.9895 79.9178) (end 126.615 79.9178) (width 0.25) (layer F.Cu) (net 4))
 (segment (start 127.265 79.6423) (end 126.9895 79.9178) (width 0.25) (layer F.Cu) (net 4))
 (segment (start 136.6597 89.4744) (end 136.6597 88.62) (width 0.25) (layer F.Cu) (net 4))
 (segment (start 136.8665 89.6812) (end 136.6597 89.4744) (width 0.25) (layer F.Cu) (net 4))
 (segment (start 138.1385 89.6812) (end 136.8665 89.6812) (width 0.25) (layer F.Cu) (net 4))
 (segment (start 139.1997 88.62) (end 138.1385 89.6812) (width 0.25) (layer F.Cu) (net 4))
 (segment (start 139.7 88.62) (end 139.1997 88.62) (width 0.25) (layer F.Cu) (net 4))
 (segment (start 137.16 88.62) (end 136.6597 88.62) (width 0.25) (layer F.Cu) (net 4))
 (segment (start 134.9349 77.8702) (end 138.5747 81.51) (width 0.25) (layer F.Cu) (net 4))
 (segment (start 131.815 77.8702) (end 134.9349 77.8702) (width 0.25) (layer F.Cu) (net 4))
 (segment (start 131.815 78.894) (end 131.815 77.8702) (width 0.25) (layer F.Cu) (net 4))
 (segment (start 142.9753 79.36) (end 140.8253 81.51) (width 0.25) (layer F.Cu) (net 4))
 (segment (start 152.32 79.36) (end 142.9753 79.36) (width 0.25) (layer F.Cu) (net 4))
 (segment (start 139.7 81.51) (end 140.8253 81.51) (width 0.25) (layer F.Cu) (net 4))
 (segment (start 139.7 81.51) (end 138.5747 81.51) (width 0.25) (layer F.Cu) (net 4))
 (segment (start 135.2695 87.2298) (end 136.6597 88.62) (width 0.25) (layer F.Cu) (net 4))
 (segment (start 129.215 87.2298) (end 135.2695 87.2298) (width 0.25) (layer F.Cu) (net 4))
 (segment (start 129.215 86.206) (end 129.215 87.2298) (width 0.25) (layer F.Cu) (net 4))
 (segment (start 124.9448 76.2) (end 119.38 76.2) (width 0.25) (layer F.Cu) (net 4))
 (segment (start 126.615 77.8702) (end 124.9448 76.2) (width 0.25) (layer F.Cu) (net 4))
 (segment (start 126.355 90.0898) (end 129.215 87.2298) (width 0.25) (layer F.Cu) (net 4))
 (segment (start 118.3609 90.0898) (end 126.355 90.0898) (width 0.25) (layer F.Cu) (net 4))
 (segment (start 117.7015 89.4304) (end 118.3609 90.0898) (width 0.25) (layer F.Cu) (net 4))
 (segment (start 117.7015 77.8785) (end 117.7015 89.4304) (width 0.25) (layer F.Cu) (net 4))
 (segment (start 119.38 76.2) (end 117.7015 77.8785) (width 0.25) (layer F.Cu) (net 4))
 (segment (start 129.865 79.8052) (end 129.865 79.9177) (width 0.25) (layer F.Cu) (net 4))
 (segment (start 129.8649 79.9178) (end 127.265 79.9178) (width 0.25) (layer F.Cu) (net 4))
 (segment (start 129.865 79.9177) (end 129.8649 79.9178) (width 0.25) (layer F.Cu) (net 4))
 (segment (start 129.8651 79.9178) (end 131.815 79.9178) (width 0.25) (layer F.Cu) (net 4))
 (segment (start 129.865 79.9177) (end 129.8651 79.9178) (width 0.25) (layer F.Cu) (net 4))
 (segment (start 131.815 78.894) (end 131.815 79.9178) (width 0.25) (layer F.Cu) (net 4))
 (segment (start 133.115 79.9344) (end 133.115 78.894) (width 0.25) (layer F.Cu) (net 10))
 (segment (start 136.6262 83.4456) (end 133.115 79.9344) (width 0.25) (layer F.Cu) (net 10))
 (segment (start 148.534 83.4456) (end 136.6262 83.4456) (width 0.25) (layer F.Cu) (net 10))
 (segment (start 151.3196 80.66) (end 148.534 83.4456) (width 0.25) (layer F.Cu) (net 10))
 (segment (start 152.32 80.66) (end 151.3196 80.66) (width 0.25) (layer F.Cu) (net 10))
 (segment (start 133.765 78.894) (end 133.765 79.9178) (width 0.25) (layer F.Cu) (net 11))
 (segment (start 136.7826 82.9354) (end 133.765 79.9178) (width 0.25) (layer F.Cu) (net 11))
 (segment (start 142.1637 82.9354) (end 136.7826 82.9354) (width 0.25) (layer F.Cu) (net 11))
 (segment (start 145.0891 80.01) (end 142.1637 82.9354) (width 0.25) (layer F.Cu) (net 11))
 (segment (start 152.32 80.01) (end 145.0891 80.01) (width 0.25) (layer F.Cu) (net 11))
 (segment (start 122.9413 86.206) (end 125.315 86.206) (width 0.25) (layer F.Cu) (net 12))
 (segment (start 120.5553 83.82) (end 122.9413 86.206) (width 0.25) (layer F.Cu) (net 12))
 (segment (start 119.38 83.82) (end 120.5553 83.82) (width 0.25) (layer F.Cu) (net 12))
 (segment (start 122.062 87.2298) (end 125.965 87.2298) (width 0.25) (layer F.Cu) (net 13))
 (segment (start 119.9961 85.1639) (end 122.062 87.2298) (width 0.25) (layer F.Cu) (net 13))
 (segment (start 118.8847 85.1639) (end 119.9961 85.1639) (width 0.25) (layer F.Cu) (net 13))
 (segment (start 118.1545 85.8941) (end 118.8847 85.1639) (width 0.25) (layer F.Cu) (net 13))
 (segment (start 118.1545 86.8665) (end 118.1545 85.8941) (width 0.25) (layer F.Cu) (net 13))
 (segment (start 119.0127 87.7247) (end 118.1545 86.8665) (width 0.25) (layer F.Cu) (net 13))
 (segment (start 119.38 87.7247) (end 119.0127 87.7247) (width 0.25) (layer F.Cu) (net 13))
 (segment (start 119.38 88.9) (end 119.38 87.7247) (width 0.25) (layer F.Cu) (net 13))
 (segment (start 125.965 86.206) (end 125.965 87.2298) (width 0.25) (layer F.Cu) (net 13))
 (segment (start 119.38 86.36) (end 120.5553 86.36) (width 0.25) (layer F.Cu) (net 15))
 (segment (start 127.915 86.206) (end 127.915 87.2298) (width 0.25) (layer F.Cu) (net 15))
 (segment (start 127.4647 87.6801) (end 127.915 87.2298) (width 0.25) (layer F.Cu) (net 15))
 (segment (start 121.8754 87.6801) (end 127.4647 87.6801) (width 0.25) (layer F.Cu) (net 15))
 (segment (start 120.5553 86.36) (end 121.8754 87.6801) (width 0.25) (layer F.Cu) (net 15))
 (segment (start 127.9018 81.269) (end 131.815 85.1822) (width 0.25) (layer F.Cu) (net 19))
 (segment (start 123.0843 81.269) (end 127.9018 81.269) (width 0.25) (layer F.Cu) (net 19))
 (segment (start 120.5553 78.74) (end 123.0843 81.269) (width 0.25) (layer F.Cu) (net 19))
 (segment (start 119.38 78.74) (end 120.5553 78.74) (width 0.25) (layer F.Cu) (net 19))
 (segment (start 131.815 86.206) (end 131.815 85.1822) (width 0.25) (layer F.Cu) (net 19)))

